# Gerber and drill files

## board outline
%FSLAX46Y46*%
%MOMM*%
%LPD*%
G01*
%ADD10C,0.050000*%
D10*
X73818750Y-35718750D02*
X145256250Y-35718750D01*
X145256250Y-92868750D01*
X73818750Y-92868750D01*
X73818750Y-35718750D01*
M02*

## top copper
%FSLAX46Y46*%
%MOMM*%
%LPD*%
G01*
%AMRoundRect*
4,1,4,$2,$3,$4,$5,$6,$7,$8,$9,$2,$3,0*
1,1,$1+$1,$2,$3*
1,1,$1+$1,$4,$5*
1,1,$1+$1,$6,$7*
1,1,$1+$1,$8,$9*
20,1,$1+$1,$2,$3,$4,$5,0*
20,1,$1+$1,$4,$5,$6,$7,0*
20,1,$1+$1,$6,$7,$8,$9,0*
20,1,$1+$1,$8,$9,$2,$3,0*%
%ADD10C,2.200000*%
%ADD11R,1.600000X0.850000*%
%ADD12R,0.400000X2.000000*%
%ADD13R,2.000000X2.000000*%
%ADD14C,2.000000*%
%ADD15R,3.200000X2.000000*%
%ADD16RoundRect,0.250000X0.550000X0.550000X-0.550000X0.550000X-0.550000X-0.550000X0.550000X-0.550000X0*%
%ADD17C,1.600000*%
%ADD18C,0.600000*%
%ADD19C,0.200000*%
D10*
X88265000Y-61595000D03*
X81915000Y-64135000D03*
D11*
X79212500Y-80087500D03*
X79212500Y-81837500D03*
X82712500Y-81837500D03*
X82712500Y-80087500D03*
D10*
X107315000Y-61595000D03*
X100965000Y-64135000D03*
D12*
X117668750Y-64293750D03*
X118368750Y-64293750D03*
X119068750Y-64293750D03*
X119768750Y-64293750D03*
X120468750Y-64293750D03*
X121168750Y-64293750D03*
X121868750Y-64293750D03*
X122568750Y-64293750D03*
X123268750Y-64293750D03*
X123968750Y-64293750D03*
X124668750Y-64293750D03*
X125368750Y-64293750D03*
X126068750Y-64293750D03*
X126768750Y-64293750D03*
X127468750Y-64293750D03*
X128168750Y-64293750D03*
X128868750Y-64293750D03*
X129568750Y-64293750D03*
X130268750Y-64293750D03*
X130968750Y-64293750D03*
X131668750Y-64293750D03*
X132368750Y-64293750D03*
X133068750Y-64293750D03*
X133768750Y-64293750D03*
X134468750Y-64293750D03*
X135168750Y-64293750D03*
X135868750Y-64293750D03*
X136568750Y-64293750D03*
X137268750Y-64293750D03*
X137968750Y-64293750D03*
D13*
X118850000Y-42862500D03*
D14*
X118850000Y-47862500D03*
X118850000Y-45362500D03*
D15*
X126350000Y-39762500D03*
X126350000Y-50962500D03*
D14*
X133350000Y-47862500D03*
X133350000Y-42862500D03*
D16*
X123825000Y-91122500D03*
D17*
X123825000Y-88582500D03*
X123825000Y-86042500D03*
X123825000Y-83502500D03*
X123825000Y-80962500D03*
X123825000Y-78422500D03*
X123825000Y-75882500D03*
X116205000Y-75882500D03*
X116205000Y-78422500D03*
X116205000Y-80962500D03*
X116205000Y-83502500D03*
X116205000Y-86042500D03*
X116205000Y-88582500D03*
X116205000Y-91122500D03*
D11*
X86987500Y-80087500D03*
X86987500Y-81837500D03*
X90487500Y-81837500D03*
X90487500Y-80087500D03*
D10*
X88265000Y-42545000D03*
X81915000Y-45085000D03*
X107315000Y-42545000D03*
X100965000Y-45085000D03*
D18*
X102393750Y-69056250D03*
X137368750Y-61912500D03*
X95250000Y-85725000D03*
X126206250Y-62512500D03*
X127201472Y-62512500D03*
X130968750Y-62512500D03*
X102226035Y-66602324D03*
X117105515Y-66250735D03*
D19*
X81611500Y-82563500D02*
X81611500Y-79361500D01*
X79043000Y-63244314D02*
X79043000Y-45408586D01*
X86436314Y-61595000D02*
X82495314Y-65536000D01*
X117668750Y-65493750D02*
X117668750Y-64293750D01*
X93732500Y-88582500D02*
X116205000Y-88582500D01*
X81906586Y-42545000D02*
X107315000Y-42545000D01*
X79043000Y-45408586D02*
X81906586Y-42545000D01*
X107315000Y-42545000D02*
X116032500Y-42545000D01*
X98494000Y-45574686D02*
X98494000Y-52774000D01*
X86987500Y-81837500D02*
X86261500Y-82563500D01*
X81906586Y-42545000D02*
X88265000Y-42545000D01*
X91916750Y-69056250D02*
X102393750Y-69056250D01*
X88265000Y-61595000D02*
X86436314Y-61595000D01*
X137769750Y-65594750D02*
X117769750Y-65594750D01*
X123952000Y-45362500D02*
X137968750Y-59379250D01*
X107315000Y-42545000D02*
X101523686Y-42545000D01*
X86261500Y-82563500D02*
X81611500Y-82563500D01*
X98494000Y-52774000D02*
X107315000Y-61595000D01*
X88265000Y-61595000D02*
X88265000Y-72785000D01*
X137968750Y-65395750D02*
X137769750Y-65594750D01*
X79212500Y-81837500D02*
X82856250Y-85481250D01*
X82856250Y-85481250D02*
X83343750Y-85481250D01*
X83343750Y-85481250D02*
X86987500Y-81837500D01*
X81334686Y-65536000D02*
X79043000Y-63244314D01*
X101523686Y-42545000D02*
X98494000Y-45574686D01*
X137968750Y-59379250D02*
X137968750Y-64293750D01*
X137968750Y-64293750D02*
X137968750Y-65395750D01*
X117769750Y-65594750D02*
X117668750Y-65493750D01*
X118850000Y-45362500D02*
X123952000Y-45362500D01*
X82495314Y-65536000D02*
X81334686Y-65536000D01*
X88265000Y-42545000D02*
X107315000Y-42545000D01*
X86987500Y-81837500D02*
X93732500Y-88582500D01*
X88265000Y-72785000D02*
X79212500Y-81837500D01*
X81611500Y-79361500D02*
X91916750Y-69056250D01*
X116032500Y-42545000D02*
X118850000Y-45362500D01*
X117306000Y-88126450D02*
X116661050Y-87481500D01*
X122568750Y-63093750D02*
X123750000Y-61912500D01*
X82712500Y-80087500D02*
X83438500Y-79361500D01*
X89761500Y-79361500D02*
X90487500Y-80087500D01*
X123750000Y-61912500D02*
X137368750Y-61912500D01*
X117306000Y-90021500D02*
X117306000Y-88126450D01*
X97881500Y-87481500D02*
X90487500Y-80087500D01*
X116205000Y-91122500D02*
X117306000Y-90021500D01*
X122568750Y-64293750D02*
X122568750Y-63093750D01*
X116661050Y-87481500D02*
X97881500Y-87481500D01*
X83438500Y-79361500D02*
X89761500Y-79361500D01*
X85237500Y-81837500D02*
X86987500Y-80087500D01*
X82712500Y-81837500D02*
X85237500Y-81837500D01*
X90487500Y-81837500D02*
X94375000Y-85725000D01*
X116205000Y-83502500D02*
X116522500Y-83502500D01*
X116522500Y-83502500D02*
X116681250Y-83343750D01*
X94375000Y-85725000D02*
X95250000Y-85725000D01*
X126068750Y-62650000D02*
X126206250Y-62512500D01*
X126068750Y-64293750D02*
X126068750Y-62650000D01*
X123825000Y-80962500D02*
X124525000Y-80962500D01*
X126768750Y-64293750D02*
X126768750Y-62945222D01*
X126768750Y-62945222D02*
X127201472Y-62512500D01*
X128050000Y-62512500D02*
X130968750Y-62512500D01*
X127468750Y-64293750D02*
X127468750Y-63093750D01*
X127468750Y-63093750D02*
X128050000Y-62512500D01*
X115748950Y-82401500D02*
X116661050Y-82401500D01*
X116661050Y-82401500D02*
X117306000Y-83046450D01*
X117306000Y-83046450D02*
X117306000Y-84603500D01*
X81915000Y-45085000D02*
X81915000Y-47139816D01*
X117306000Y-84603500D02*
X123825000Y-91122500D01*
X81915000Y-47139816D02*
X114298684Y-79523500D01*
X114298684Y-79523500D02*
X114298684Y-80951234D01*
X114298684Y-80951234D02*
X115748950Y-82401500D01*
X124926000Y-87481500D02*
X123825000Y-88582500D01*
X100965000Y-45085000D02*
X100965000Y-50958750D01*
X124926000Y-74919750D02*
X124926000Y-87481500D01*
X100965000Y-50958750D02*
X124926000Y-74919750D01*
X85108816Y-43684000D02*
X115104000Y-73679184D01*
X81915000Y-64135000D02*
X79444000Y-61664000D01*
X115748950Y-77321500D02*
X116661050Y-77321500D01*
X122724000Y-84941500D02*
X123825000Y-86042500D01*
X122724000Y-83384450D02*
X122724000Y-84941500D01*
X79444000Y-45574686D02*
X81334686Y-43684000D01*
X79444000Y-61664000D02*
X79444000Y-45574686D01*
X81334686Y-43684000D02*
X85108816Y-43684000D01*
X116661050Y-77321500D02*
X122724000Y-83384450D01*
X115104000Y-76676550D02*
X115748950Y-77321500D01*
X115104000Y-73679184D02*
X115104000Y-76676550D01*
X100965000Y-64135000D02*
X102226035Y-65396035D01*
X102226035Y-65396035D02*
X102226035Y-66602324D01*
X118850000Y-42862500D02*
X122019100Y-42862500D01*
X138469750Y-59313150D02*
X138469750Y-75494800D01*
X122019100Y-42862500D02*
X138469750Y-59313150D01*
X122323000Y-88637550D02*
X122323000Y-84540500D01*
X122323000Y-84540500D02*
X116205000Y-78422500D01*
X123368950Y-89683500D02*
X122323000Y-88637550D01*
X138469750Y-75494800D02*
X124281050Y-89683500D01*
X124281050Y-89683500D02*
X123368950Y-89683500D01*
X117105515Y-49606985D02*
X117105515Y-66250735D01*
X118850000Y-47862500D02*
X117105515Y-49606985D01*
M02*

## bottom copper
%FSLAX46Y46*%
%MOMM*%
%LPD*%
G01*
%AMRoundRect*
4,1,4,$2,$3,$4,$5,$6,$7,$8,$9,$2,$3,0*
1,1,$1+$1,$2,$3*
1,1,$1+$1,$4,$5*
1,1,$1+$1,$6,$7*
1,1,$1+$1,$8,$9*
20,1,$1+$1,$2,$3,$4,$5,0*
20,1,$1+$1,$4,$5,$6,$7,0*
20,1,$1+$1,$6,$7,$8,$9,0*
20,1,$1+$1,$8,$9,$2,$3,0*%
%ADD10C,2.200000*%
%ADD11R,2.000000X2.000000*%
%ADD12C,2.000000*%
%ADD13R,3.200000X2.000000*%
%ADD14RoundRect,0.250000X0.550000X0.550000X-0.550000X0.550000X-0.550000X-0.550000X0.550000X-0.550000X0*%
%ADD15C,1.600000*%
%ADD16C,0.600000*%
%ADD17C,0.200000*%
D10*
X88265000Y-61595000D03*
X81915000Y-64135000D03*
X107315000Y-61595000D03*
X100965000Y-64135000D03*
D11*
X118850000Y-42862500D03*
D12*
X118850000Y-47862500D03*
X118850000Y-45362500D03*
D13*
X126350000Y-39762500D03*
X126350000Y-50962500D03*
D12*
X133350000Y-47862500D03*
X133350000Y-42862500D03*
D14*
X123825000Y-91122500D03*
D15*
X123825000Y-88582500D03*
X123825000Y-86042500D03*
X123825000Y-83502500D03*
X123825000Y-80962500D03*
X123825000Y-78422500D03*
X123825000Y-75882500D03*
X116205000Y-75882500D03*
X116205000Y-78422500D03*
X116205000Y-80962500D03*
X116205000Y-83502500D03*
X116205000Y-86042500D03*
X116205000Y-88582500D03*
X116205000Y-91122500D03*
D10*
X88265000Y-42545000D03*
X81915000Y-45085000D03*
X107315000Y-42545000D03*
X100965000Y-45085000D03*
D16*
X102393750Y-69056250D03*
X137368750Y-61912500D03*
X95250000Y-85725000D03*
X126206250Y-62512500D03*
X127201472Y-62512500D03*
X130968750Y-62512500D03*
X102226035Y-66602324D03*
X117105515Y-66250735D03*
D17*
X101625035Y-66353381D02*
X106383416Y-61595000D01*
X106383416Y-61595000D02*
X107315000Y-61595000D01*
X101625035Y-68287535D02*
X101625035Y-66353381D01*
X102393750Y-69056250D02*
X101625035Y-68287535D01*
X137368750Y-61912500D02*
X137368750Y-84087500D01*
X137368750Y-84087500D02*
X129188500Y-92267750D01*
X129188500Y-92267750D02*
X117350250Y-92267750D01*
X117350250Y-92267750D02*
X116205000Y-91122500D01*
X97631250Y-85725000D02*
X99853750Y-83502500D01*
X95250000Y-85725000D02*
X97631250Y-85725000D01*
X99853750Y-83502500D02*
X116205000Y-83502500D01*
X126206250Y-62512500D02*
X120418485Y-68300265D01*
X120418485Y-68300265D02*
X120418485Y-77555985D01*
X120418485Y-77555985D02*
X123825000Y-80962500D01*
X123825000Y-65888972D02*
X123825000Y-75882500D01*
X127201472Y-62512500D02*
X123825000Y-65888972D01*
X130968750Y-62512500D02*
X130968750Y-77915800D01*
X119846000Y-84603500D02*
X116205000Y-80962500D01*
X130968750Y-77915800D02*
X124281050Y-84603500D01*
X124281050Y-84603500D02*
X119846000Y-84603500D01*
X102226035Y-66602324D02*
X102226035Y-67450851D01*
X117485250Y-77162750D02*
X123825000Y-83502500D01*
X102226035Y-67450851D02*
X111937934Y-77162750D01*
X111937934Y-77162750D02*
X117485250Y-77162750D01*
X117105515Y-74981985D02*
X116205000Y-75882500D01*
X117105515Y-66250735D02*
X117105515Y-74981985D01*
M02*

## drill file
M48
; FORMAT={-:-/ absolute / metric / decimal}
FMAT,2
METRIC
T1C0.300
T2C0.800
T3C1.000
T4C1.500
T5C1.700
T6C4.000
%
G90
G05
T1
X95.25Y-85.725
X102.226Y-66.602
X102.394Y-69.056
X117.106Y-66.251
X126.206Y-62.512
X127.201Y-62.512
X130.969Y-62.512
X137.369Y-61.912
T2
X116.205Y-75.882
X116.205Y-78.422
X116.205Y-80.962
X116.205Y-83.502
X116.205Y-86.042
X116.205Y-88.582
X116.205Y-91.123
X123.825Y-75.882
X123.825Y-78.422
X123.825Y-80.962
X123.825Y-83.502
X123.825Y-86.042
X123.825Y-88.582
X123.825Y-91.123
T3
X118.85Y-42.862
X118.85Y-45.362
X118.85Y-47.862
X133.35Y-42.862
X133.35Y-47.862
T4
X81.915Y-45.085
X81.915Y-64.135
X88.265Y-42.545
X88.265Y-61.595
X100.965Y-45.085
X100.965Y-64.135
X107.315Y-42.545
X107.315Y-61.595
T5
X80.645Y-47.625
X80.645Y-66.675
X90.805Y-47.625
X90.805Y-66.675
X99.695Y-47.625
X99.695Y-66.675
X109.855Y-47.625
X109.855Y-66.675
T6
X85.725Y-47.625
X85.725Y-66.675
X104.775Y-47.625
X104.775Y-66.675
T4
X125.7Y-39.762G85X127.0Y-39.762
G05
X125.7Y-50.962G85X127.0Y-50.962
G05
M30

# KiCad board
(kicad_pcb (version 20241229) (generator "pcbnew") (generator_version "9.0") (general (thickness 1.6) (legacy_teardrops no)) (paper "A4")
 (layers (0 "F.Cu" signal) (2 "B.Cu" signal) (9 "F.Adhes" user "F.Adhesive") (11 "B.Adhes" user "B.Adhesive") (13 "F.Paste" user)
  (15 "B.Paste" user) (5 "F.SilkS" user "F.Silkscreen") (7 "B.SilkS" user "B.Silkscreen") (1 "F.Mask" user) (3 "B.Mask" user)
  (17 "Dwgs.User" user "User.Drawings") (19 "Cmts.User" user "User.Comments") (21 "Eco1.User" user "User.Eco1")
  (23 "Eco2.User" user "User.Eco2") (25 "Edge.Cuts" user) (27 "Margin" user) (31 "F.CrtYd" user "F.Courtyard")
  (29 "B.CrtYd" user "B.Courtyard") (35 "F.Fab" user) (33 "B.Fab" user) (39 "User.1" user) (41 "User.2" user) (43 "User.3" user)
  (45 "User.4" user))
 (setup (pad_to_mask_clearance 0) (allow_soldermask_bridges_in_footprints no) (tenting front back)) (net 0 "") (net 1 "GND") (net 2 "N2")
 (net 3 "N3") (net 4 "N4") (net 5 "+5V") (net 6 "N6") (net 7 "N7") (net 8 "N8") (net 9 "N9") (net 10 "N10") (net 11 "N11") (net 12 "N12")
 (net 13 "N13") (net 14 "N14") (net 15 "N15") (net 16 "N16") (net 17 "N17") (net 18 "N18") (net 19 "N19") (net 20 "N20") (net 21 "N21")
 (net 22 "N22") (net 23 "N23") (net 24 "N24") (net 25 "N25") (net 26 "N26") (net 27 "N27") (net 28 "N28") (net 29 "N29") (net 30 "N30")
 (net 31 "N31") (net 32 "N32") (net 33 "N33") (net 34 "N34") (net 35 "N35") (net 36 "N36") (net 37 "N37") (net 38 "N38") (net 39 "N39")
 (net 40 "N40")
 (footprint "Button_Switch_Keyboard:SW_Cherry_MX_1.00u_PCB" (layer "F.Cu") (at 88.265 61.595)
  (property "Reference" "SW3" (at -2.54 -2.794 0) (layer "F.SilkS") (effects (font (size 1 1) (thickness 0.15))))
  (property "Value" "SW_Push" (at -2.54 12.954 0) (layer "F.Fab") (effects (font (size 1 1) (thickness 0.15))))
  (pad "" np_thru_hole circle (at -7.62 5.08) (size 1.7 1.7) (drill 1.7) (layers "*.Cu" "*.Mask"))
  (pad "" np_thru_hole circle (at -2.54 5.08) (size 4 4) (drill 4) (layers "*.Cu" "*.Mask"))
  (pad "" np_thru_hole circle (at 2.54 5.08) (size 1.7 1.7) (drill 1.7) (layers "*.Cu" "*.Mask"))
  (pad "1" thru_hole circle (at 0 0) (size 2.2 2.2) (drill 1.5) (layers "*.Cu" "*.Mask") (remove_unused_layers no) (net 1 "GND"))
  (pad "2" thru_hole circle (at -6.35 2.54) (size 2.2 2.2) (drill 1.5) (layers "*.Cu" "*.Mask") (remove_unused_layers no) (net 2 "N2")))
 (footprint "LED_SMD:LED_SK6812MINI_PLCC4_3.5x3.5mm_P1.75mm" (layer "F.Cu") (at 80.9625 80.9625)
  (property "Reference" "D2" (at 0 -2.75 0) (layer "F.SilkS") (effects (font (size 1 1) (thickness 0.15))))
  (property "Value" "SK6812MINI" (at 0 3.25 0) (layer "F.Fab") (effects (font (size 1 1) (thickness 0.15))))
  (pad "1" smd rect (at -1.75 -0.875) (size 1.6 0.85) (layers "F.Cu" "F.Mask" "F.Paste") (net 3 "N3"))
  (pad "2" smd rect (at -1.75 0.875) (size 1.6 0.85) (layers "F.Cu" "F.Mask" "F.Paste") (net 1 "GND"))
  (pad "3" smd rect (at 1.75 0.875) (size 1.6 0.85) (layers "F.Cu" "F.Mask" "F.Paste") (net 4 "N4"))
  (pad "4" smd rect (at 1.75 -0.875) (size 1.6 0.85) (layers "F.Cu" "F.Mask" "F.Paste") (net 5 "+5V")))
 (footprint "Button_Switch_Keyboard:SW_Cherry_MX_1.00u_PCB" (layer "F.Cu") (at 107.315 61.595)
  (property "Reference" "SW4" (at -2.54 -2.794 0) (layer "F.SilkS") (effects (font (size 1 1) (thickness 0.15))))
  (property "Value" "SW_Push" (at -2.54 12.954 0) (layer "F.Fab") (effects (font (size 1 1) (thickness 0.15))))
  (pad "" np_thru_hole circle (at -7.62 5.08) (size 1.7 1.7) (drill 1.7) (layers "*.Cu" "*.Mask"))
  (pad "" np_thru_hole circle (at -2.54 5.08) (size 4 4) (drill 4) (layers "*.Cu" "*.Mask"))
  (pad "" np_thru_hole circle (at 2.54 5.08) (size 1.7 1.7) (drill 1.7) (layers "*.Cu" "*.Mask"))
  (pad "1" thru_hole circle (at 0 0) (size 2.2 2.2) (drill 1.5) (layers "*.Cu" "*.Mask") (remove_unused_layers no) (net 1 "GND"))
  (pad "2" thru_hole circle (at -6.35 2.54) (size 2.2 2.2) (drill 1.5) (layers "*.Cu" "*.Mask") (remove_unused_layers no) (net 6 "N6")))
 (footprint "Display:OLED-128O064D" (layer "F.Cu") (at 127.81875 64.29375)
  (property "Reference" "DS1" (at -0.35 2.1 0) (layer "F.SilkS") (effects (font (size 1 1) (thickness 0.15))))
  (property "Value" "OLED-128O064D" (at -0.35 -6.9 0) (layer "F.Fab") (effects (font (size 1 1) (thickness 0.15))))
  (pad "1" smd rect (at -10.15 0) (size 0.4 2) (layers "F.Cu" "F.Mask" "F.Paste") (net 1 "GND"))
  (pad "2" smd rect (at -9.45 0) (size 0.4 2) (layers "F.Cu" "F.Mask" "F.Paste") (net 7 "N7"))
  (pad "3" smd rect (at -8.75 0) (size 0.4 2) (layers "F.Cu" "F.Mask" "F.Paste") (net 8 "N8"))
  (pad "4" smd rect (at -8.05 0) (size 0.4 2) (layers "F.Cu" "F.Mask" "F.Paste") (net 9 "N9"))
  (pad "5" smd rect (at -7.35 0) (size 0.4 2) (layers "F.Cu" "F.Mask" "F.Paste") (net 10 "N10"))
  (pad "6" smd rect (at -6.65 0) (size 0.4 2) (layers "F.Cu" "F.Mask" "F.Paste") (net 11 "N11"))
  (pad "7" smd rect (at -5.95 0) (size 0.4 2) (layers "F.Cu" "F.Mask" "F.Paste") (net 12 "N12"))
  (pad "8" smd rect (at -5.25 0) (size 0.4 2) (layers "F.Cu" "F.Mask" "F.Paste") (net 5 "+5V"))
  (pad "9" smd rect (at -4.55 0) (size 0.4 2) (layers "F.Cu" "F.Mask" "F.Paste") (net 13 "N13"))
  (pad "10" smd rect (at -3.85 0) (size 0.4 2) (layers "F.Cu" "F.Mask" "F.Paste") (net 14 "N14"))
  (pad "11" smd rect (at -3.15 0) (size 0.4 2) (layers "F.Cu" "F.Mask" "F.Paste") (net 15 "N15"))
  (pad "12" smd rect (at -2.45 0) (size 0.4 2) (layers "F.Cu" "F.Mask" "F.Paste") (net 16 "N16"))
  (pad "13" smd rect (at -1.75 0) (size 0.4 2) (layers "F.Cu" "F.Mask" "F.Paste") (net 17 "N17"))
  (pad "14" smd rect (at -1.05 0) (size 0.4 2) (layers "F.Cu" "F.Mask" "F.Paste") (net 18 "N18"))
  (pad "15" smd rect (at -0.35 0) (size 0.4 2) (layers "F.Cu" "F.Mask" "F.Paste") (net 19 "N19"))
  (pad "16" smd rect (at 0.35 0) (size 0.4 2) (layers "F.Cu" "F.Mask" "F.Paste") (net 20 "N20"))
  (pad "17" smd rect (at 1.05 0) (size 0.4 2) (layers "F.Cu" "F.Mask" "F.Paste") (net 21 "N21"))
  (pad "18" smd rect (at 1.75 0) (size 0.4 2) (layers "F.Cu" "F.Mask" "F.Paste") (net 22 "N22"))
  (pad "19" smd rect (at 2.45 0) (size 0.4 2) (layers "F.Cu" "F.Mask" "F.Paste") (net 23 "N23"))
  (pad "20" smd rect (at 3.15 0) (size 0.4 2) (layers "F.Cu" "F.Mask" "F.Paste") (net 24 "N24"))
  (pad "21" smd rect (at 3.85 0) (size 0.4 2) (layers "F.Cu" "F.Mask" "F.Paste") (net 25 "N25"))
  (pad "22" smd rect (at 4.55 0) (size 0.4 2) (layers "F.Cu" "F.Mask" "F.Paste") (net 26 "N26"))
  (pad "23" smd rect (at 5.25 0) (size 0.4 2) (layers "F.Cu" "F.Mask" "F.Paste") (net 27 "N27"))
  (pad "24" smd rect (at 5.95 0) (size 0.4 2) (layers "F.Cu" "F.Mask" "F.Paste") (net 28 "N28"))
  (pad "25" smd rect (at 6.65 0) (size 0.4 2) (layers "F.Cu" "F.Mask" "F.Paste") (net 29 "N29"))
  (pad "26" smd rect (at 7.35 0) (size 0.4 2) (layers "F.Cu" "F.Mask" "F.Paste") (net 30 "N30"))
  (pad "27" smd rect (at 8.05 0) (size 0.4 2) (layers "F.Cu" "F.Mask" "F.Paste") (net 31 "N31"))
  (pad "28" smd rect (at 8.75 0) (size 0.4 2) (layers "F.Cu" "F.Mask" "F.Paste") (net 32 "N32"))
  (pad "29" smd rect (at 9.45 0) (size 0.4 2) (layers "F.Cu" "F.Mask" "F.Paste") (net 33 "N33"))
  (pad "30" smd rect (at 10.15 0) (size 0.4 2) (layers "F.Cu" "F.Mask" "F.Paste") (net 1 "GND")))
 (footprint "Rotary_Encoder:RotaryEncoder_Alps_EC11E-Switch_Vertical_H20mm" (layer "F.Cu") (at 118.85 42.8625)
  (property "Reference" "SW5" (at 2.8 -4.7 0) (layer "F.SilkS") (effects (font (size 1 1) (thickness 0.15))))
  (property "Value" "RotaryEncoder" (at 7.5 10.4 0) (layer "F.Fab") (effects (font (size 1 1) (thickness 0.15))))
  (pad "A" thru_hole rect (at 0 0) (size 2 2) (drill 1) (layers "*.Cu" "*.Mask") (remove_unused_layers no) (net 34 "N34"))
  (pad "B" thru_hole circle (at 0 5) (size 2 2) (drill 1) (layers "*.Cu" "*.Mask") (remove_unused_layers no) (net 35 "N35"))
  (pad "C" thru_hole circle (at 0 2.5) (size 2 2) (drill 1) (layers "*.Cu" "*.Mask") (remove_unused_layers no) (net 1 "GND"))
  (pad "MP" thru_hole rect (at 7.5 -3.1) (size 3.2 2) (drill oval 2.8 1.5) (layers "*.Cu" "*.Mask") (remove_unused_layers no))
  (pad "MP" thru_hole rect (at 7.5 8.1) (size 3.2 2) (drill oval 2.8 1.5) (layers "*.Cu" "*.Mask") (remove_unused_layers no))
  (pad "S1" thru_hole circle (at 14.5 5) (size 2 2) (drill 1) (layers "*.Cu" "*.Mask") (remove_unused_layers no))
  (pad "S2" thru_hole circle (at 14.5 0) (size 2 2) (drill 1) (layers "*.Cu" "*.Mask") (remove_unused_layers no)))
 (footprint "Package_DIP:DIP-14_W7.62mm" (layer "F.Cu") (at 123.825 91.1225 180)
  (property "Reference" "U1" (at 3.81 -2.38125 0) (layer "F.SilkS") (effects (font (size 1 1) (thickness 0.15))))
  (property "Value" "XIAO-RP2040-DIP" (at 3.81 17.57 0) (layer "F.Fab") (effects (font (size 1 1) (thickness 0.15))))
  (pad "1" thru_hole roundrect (at 0 0 180) (size 1.6 1.6) (drill 0.8) (layers "*.Cu" "*.Mask") (remove_unused_layers no)
   (roundrect_rratio 0.15625) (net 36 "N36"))
  (pad "2" thru_hole circle (at 0 2.54 180) (size 1.6 1.6) (drill 0.8) (layers "*.Cu" "*.Mask") (remove_unused_layers no) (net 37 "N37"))
  (pad "3" thru_hole circle (at 0 5.08 180) (size 1.6 1.6) (drill 0.8) (layers "*.Cu" "*.Mask") (remove_unused_layers no) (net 2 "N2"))
  (pad "4" thru_hole circle (at 0 7.62 180) (size 1.6 1.6) (drill 0.8) (layers "*.Cu" "*.Mask") (remove_unused_layers no) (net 6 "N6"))
  (pad "5" thru_hole circle (at 0 10.16 180) (size 1.6 1.6) (drill 0.8) (layers "*.Cu" "*.Mask") (remove_unused_layers no) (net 17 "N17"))
  (pad "6" thru_hole circle (at 0 12.7 180) (size 1.6 1.6) (drill 0.8) (layers "*.Cu" "*.Mask") (remove_unused_layers no) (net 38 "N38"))
  (pad "7" thru_hole circle (at 0 15.24 180) (size 1.6 1.6) (drill 0.8) (layers "*.Cu" "*.Mask") (remove_unused_layers no) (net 18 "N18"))
  (pad "8" thru_hole circle (at 7.62 15.24 180) (size 1.6 1.6) (drill 0.8) (layers "*.Cu" "*.Mask") (remove_unused_layers no) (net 35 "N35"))
  (pad "9" thru_hole circle (at 7.62 12.7 180) (size 1.6 1.6) (drill 0.8) (layers "*.Cu" "*.Mask") (remove_unused_layers no) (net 34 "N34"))
  (pad "10" thru_hole circle (at 7.62 10.16 180) (size 1.6 1.6) (drill 0.8) (layers "*.Cu" "*.Mask") (remove_unused_layers no)
   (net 19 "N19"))
  (pad "11" thru_hole circle (at 7.62 7.62 180) (size 1.6 1.6) (drill 0.8) (layers "*.Cu" "*.Mask") (remove_unused_layers no) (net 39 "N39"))
  (pad "12" thru_hole circle (at 7.62 5.08 180) (size 1.6 1.6) (drill 0.8) (layers "*.Cu" "*.Mask") (remove_unused_layers no) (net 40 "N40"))
  (pad "13" thru_hole circle (at 7.62 2.54 180) (size 1.6 1.6) (drill 0.8) (layers "*.Cu" "*.Mask") (remove_unused_layers no) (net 1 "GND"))
  (pad "14" thru_hole circle (at 7.62 0 180) (size 1.6 1.6) (drill 0.8) (layers "*.Cu" "*.Mask") (remove_unused_layers no) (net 5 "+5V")))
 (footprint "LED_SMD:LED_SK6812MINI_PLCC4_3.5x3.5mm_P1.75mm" (layer "F.Cu") (at 88.7375 80.9625)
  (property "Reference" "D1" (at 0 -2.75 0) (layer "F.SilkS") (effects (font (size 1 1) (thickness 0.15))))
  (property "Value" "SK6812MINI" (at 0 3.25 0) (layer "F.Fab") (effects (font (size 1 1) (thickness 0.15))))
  (pad "1" smd rect (at -1.75 -0.875) (size 1.6 0.85) (layers "F.Cu" "F.Mask" "F.Paste") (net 4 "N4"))
  (pad "2" smd rect (at -1.75 0.875) (size 1.6 0.85) (layers "F.Cu" "F.Mask" "F.Paste") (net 1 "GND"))
  (pad "3" smd rect (at 1.75 0.875) (size 1.6 0.85) (layers "F.Cu" "F.Mask" "F.Paste") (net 39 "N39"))
  (pad "4" smd rect (at 1.75 -0.875) (size 1.6 0.85) (layers "F.Cu" "F.Mask" "F.Paste") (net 5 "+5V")))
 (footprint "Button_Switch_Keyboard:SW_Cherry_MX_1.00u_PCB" (layer "F.Cu") (at 88.265 42.545)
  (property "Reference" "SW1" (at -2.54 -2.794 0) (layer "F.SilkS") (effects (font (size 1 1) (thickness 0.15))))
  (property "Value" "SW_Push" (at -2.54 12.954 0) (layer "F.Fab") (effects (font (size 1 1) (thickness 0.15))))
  (pad "" np_thru_hole circle (at -7.62 5.08) (size 1.7 1.7) (drill 1.7) (layers "*.Cu" "*.Mask"))
  (pad "" np_thru_hole circle (at -2.54 5.08) (size 4 4) (drill 4) (layers "*.Cu" "*.Mask"))
  (pad "" np_thru_hole circle (at 2.54 5.08) (size 1.7 1.7) (drill 1.7) (layers "*.Cu" "*.Mask"))
  (pad "1" thru_hole circle (at 0 0) (size 2.2 2.2) (drill 1.5) (layers "*.Cu" "*.Mask") (remove_unused_layers no) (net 1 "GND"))
  (pad "2" thru_hole circle (at -6.35 2.54) (size 2.2 2.2) (drill 1.5) (layers "*.Cu" "*.Mask") (remove_unused_layers no) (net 36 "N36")))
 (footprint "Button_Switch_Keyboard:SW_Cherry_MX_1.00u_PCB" (layer "F.Cu") (at 107.315 42.545)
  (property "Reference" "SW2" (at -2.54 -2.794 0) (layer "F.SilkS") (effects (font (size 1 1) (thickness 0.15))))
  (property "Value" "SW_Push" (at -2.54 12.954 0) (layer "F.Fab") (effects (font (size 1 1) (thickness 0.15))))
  (pad "" np_thru_hole circle (at -7.62 5.08) (size 1.7 1.7) (drill 1.7) (layers "*.Cu" "*.Mask"))
  (pad "" np_thru_hole circle (at -2.54 5.08) (size 4 4) (drill 4) (layers "*.Cu" "*.Mask"))
  (pad "" np_thru_hole circle (at 2.54 5.08) (size 1.7 1.7) (drill 1.7) (layers "*.Cu" "*.Mask"))
  (pad "1" thru_hole circle (at 0 0) (size 2.2 2.2) (drill 1.5) (layers "*.Cu" "*.Mask") (remove_unused_layers no) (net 1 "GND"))
  (pad "2" thru_hole circle (at -6.35 2.54) (size 2.2 2.2) (drill 1.5) (layers "*.Cu" "*.Mask") (remove_unused_layers no) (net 37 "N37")))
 (gr_rect (start 73.81875 35.71875) (end 145.25625 92.86875) (stroke (width 0.05) (type default)) (fill no) (layer "Edge.Cuts"))
 (segment (start 81.6115 82.5635) (end 81.6115 79.3615) (width 0.2) (layer "F.Cu") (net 1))
 (segment (start 79.043 63.244314) (end 79.043 45.408586) (width 0.2) (layer "F.Cu") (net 1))
 (segment (start 86.436314 61.595) (end 82.495314 65.536) (width 0.2) (layer "F.Cu") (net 1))
 (segment (start 117.66875 65.49375) (end 117.66875 64.29375) (width 0.2) (layer "F.Cu") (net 1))
 (segment (start 93.7325 88.5825) (end 116.205 88.5825) (width 0.2) (layer "F.Cu") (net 1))
 (segment (start 81.906586 42.545) (end 107.315 42.545) (width 0.2) (layer "F.Cu") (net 1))
 (segment (start 79.043 45.408586) (end 81.906586 42.545) (width 0.2) (layer "F.Cu") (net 1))
 (segment (start 107.315 42.545) (end 116.0325 42.545) (width 0.2) (layer "F.Cu") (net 1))
 (segment (start 98.494 45.574686) (end 98.494 52.774) (width 0.2) (layer "F.Cu") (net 1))
 (segment (start 86.9875 81.8375) (end 86.2615 82.5635) (width 0.2) (layer "F.Cu") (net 1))
 (segment (start 81.906586 42.545) (end 88.265 42.545) (width 0.2) (layer "F.Cu") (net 1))
 (segment (start 91.91675 69.05625) (end 102.39375 69.05625) (width 0.2) (layer "F.Cu") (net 1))
 (segment (start 88.265 61.595) (end 86.436314 61.595) (width 0.2) (layer "F.Cu") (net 1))
 (segment (start 137.76975 65.59475) (end 117.76975 65.59475) (width 0.2) (layer "F.Cu") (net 1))
 (segment (start 123.952 45.3625) (end 137.96875 59.37925) (width 0.2) (layer "F.Cu") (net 1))
 (segment (start 107.315 42.545) (end 101.523686 42.545) (width 0.2) (layer "F.Cu") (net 1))
 (segment (start 86.2615 82.5635) (end 81.6115 82.5635) (width 0.2) (layer "F.Cu") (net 1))
 (segment (start 98.494 52.774) (end 107.315 61.595) (width 0.2) (layer "F.Cu") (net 1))
 (segment (start 88.265 61.595) (end 88.265 72.785) (width 0.2) (layer "F.Cu") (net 1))
 (segment (start 137.96875 65.39575) (end 137.76975 65.59475) (width 0.2) (layer "F.Cu") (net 1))
 (segment (start 79.2125 81.8375) (end 82.85625 85.48125) (width 0.2) (layer "F.Cu") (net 1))
 (segment (start 82.85625 85.48125) (end 83.34375 85.48125) (width 0.2) (layer "F.Cu") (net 1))
 (segment (start 83.34375 85.48125) (end 86.9875 81.8375) (width 0.2) (layer "F.Cu") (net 1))
 (segment (start 81.334686 65.536) (end 79.043 63.244314) (width 0.2) (layer "F.Cu") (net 1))
 (segment (start 101.523686 42.545) (end 98.494 45.574686) (width 0.2) (layer "F.Cu") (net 1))
 (segment (start 137.96875 59.37925) (end 137.96875 64.29375) (width 0.2) (layer "F.Cu") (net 1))
 (segment (start 137.96875 64.29375) (end 137.96875 65.39575) (width 0.2) (layer "F.Cu") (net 1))
 (segment (start 117.76975 65.59475) (end 117.66875 65.49375) (width 0.2) (layer "F.Cu") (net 1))
 (segment (start 118.85 45.3625) (end 123.952 45.3625) (width 0.2) (layer "F.Cu") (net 1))
 (segment (start 82.495314 65.536) (end 81.334686 65.536) (width 0.2) (layer "F.Cu") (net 1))
 (segment (start 88.265 42.545) (end 107.315 42.545) (width 0.2) (layer "F.Cu") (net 1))
 (segment (start 86.9875 81.8375) (end 93.7325 88.5825) (width 0.2) (layer "F.Cu") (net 1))
 (segment (start 88.265 72.785) (end 79.2125 81.8375) (width 0.2) (layer "F.Cu") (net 1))
 (segment (start 81.6115 79.3615) (end 91.91675 69.05625) (width 0.2) (layer "F.Cu") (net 1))
 (segment (start 116.0325 42.545) (end 118.85 45.3625) (width 0.2) (layer "F.Cu") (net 1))
 (via (at 102.39375 69.05625) (size 0.6) (drill 0.3) (layers "F.Cu" "B.Cu") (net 1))
 (segment (start 101.625035 66.353381) (end 106.383416 61.595) (width 0.2) (layer "B.Cu") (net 1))
 (segment (start 106.383416 61.595) (end 107.315 61.595) (width 0.2) (layer "B.Cu") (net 1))
 (segment (start 101.625035 68.287535) (end 101.625035 66.353381) (width 0.2) (layer "B.Cu") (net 1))
 (segment (start 102.39375 69.05625) (end 101.625035 68.287535) (width 0.2) (layer "B.Cu") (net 1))
 (segment (start 117.306 88.12645) (end 116.66105 87.4815) (width 0.2) (layer "F.Cu") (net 5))
 (segment (start 122.56875 63.09375) (end 123.75 61.9125) (width 0.2) (layer "F.Cu") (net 5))
 (segment (start 82.7125 80.0875) (end 83.4385 79.3615) (width 0.2) (layer "F.Cu") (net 5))
 (segment (start 89.7615 79.3615) (end 90.4875 80.0875) (width 0.2) (layer "F.Cu") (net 5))
 (segment (start 123.75 61.9125) (end 137.36875 61.9125) (width 0.2) (layer "F.Cu") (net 5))
 (segment (start 117.306 90.0215) (end 117.306 88.12645) (width 0.2) (layer "F.Cu") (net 5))
 (segment (start 97.8815 87.4815) (end 90.4875 80.0875) (width 0.2) (layer "F.Cu") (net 5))
 (segment (start 116.205 91.1225) (end 117.306 90.0215) (width 0.2) (layer "F.Cu") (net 5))
 (segment (start 122.56875 64.29375) (end 122.56875 63.09375) (width 0.2) (layer "F.Cu") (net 5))
 (segment (start 116.66105 87.4815) (end 97.8815 87.4815) (width 0.2) (layer "F.Cu") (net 5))
 (segment (start 83.4385 79.3615) (end 89.7615 79.3615) (width 0.2) (layer "F.Cu") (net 5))
 (via (at 137.36875 61.9125) (size 0.6) (drill 0.3) (layers "F.Cu" "B.Cu") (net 5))
 (segment (start 137.36875 61.9125) (end 137.36875 84.0875) (width 0.2) (layer "B.Cu") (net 5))
 (segment (start 137.36875 84.0875) (end 129.1885 92.26775) (width 0.2) (layer "B.Cu") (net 5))
 (segment (start 129.1885 92.26775) (end 117.35025 92.26775) (width 0.2) (layer "B.Cu") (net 5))
 (segment (start 117.35025 92.26775) (end 116.205 91.1225) (width 0.2) (layer "B.Cu") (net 5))
 (segment (start 85.2375 81.8375) (end 86.9875 80.0875) (width 0.2) (layer "F.Cu") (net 4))
 (segment (start 82.7125 81.8375) (end 85.2375 81.8375) (width 0.2) (layer "F.Cu") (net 4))
 (segment (start 90.4875 81.8375) (end 94.375 85.725) (width 0.2) (layer "F.Cu") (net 39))
 (segment (start 116.205 83.5025) (end 116.5225 83.5025) (width 0.2) (layer "F.Cu") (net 39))
 (segment (start 116.5225 83.5025) (end 116.68125 83.34375) (width 0.2) (layer "F.Cu") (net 39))
 (segment (start 94.375 85.725) (end 95.25 85.725) (width 0.2) (layer "F.Cu") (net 39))
 (via (at 95.25 85.725) (size 0.6) (drill 0.3) (layers "F.Cu" "B.Cu") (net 39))
 (segment (start 97.63125 85.725) (end 99.85375 83.5025) (width 0.2) (layer "B.Cu") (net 39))
 (segment (start 95.25 85.725) (end 97.63125 85.725) (width 0.2) (layer "B.Cu") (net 39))
 (segment (start 99.85375 83.5025) (end 116.205 83.5025) (width 0.2) (layer "B.Cu") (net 39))
 (segment (start 126.06875 62.65) (end 126.20625 62.5125) (width 0.2) (layer "F.Cu") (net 17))
 (segment (start 126.06875 64.29375) (end 126.06875 62.65) (width 0.2) (layer "F.Cu") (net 17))
 (segment (start 123.825 80.9625) (end 124.525 80.9625) (width 0.2) (layer "F.Cu") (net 17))
 (via (at 126.20625 62.5125) (size 0.6) (drill 0.3) (layers "F.Cu" "B.Cu") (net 17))
 (segment (start 126.20625 62.5125) (end 120.418485 68.300265) (width 0.2) (layer "B.Cu") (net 17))
 (segment (start 120.418485 68.300265) (end 120.418485 77.555985) (width 0.2) (layer "B.Cu") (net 17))
 (segment (start 120.418485 77.555985) (end 123.825 80.9625) (width 0.2) (layer "B.Cu") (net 17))
 (segment (start 126.76875 64.29375) (end 126.76875 62.945222) (width 0.2) (layer "F.Cu") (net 18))
 (segment (start 126.76875 62.945222) (end 127.201472 62.5125) (width 0.2) (layer "F.Cu") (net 18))
 (via (at 127.201472 62.5125) (size 0.6) (drill 0.3) (layers "F.Cu" "B.Cu") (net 18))
 (segment (start 123.825 65.888972) (end 123.825 75.8825) (width 0.2) (layer "B.Cu") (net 18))
 (segment (start 127.201472 62.5125) (end 123.825 65.888972) (width 0.2) (layer "B.Cu") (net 18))
 (segment (start 128.05 62.5125) (end 130.96875 62.5125) (width 0.2) (layer "F.Cu") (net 19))
 (segment (start 127.46875 64.29375) (end 127.46875 63.09375) (width 0.2) (layer "F.Cu") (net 19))
 (segment (start 127.46875 63.09375) (end 128.05 62.5125) (width 0.2) (layer "F.Cu") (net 19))
 (via (at 130.96875 62.5125) (size 0.6) (drill 0.3) (layers "F.Cu" "B.Cu") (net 19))
 (segment (start 130.96875 62.5125) (end 130.96875 77.9158) (width 0.2) (layer "B.Cu") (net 19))
 (segment (start 119.846 84.6035) (end 116.205 80.9625) (width 0.2) (layer "B.Cu") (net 19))
 (segment (start 130.96875 77.9158) (end 124.28105 84.6035) (width 0.2) (layer "B.Cu") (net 19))
 (segment (start 124.28105 84.6035) (end 119.846 84.6035) (width 0.2) (layer "B.Cu") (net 19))
 (segment (start 115.74895 82.4015) (end 116.66105 82.4015) (width 0.2) (layer "F.Cu") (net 36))
 (segment (start 116.66105 82.4015) (end 117.306 83.04645) (width 0.2) (layer "F.Cu") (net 36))
 (segment (start 117.306 83.04645) (end 117.306 84.6035) (width 0.2) (layer "F.Cu") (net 36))
 (segment (start 81.915 45.085) (end 81.915 47.139816) (width 0.2) (layer "F.Cu") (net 36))
 (segment (start 117.306 84.6035) (end 123.825 91.1225) (width 0.2) (layer "F.Cu") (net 36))
 (segment (start 81.915 47.139816) (end 114.298684 79.5235) (width 0.2) (layer "F.Cu") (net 36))
 (segment (start 114.298684 79.5235) (end 114.298684 80.951234) (width 0.2) (layer "F.Cu") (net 36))
 (segment (start 114.298684 80.951234) (end 115.74895 82.4015) (width 0.2) (layer "F.Cu") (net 36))
 (segment (start 124.926 87.4815) (end 123.825 88.5825) (width 0.2) (layer "F.Cu") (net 37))
 (segment (start 100.965 45.085) (end 100.965 50.95875) (width 0.2) (layer "F.Cu") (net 37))
 (segment (start 124.926 74.91975) (end 124.926 87.4815) (width 0.2) (layer "F.Cu") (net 37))
 (segment (start 100.965 50.95875) (end 124.926 74.91975) (width 0.2) (layer "F.Cu") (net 37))
 (segment (start 85.108816 43.684) (end 115.104 73.679184) (width 0.2) (layer "F.Cu") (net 2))
 (segment (start 81.915 64.135) (end 79.444 61.664) (width 0.2) (layer "F.Cu") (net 2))
 (segment (start 115.74895 77.3215) (end 116.66105 77.3215) (width 0.2) (layer "F.Cu") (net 2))
 (segment (start 122.724 84.9415) (end 123.825 86.0425) (width 0.2) (layer "F.Cu") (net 2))
 (segment (start 122.724 83.38445) (end 122.724 84.9415) (width 0.2) (layer "F.Cu") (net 2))
 (segment (start 79.444 45.574686) (end 81.334686 43.684) (width 0.2) (layer "F.Cu") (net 2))
 (segment (start 79.444 61.664) (end 79.444 45.574686) (width 0.2) (layer "F.Cu") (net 2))
 (segment (start 81.334686 43.684) (end 85.108816 43.684) (width 0.2) (layer "F.Cu") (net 2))
 (segment (start 116.66105 77.3215) (end 122.724 83.38445) (width 0.2) (layer "F.Cu") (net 2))
 (segment (start 115.104 76.67655) (end 115.74895 77.3215) (width 0.2) (layer "F.Cu") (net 2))
 (segment (start 115.104 73.679184) (end 115.104 76.67655) (width 0.2) (layer "F.Cu") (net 2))
 (segment (start 100.965 64.135) (end 102.226035 65.396035) (width 0.2) (layer "F.Cu") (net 6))
 (segment (start 102.226035 65.396035) (end 102.226035 66.602324) (width 0.2) (layer "F.Cu") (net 6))
 (via (at 102.226035 66.602324) (size 0.6) (drill 0.3) (layers "F.Cu" "B.Cu") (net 6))
 (segment (start 102.226035 66.602324) (end 102.226035 67.450851) (width 0.2) (layer "B.Cu") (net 6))
 (segment (start 117.48525 77.16275) (end 123.825 83.5025) (width 0.2) (layer "B.Cu") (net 6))
 (segment (start 102.226035 67.450851) (end 111.937934 77.16275) (width 0.2) (layer "B.Cu") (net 6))
 (segment (start 111.937934 77.16275) (end 117.48525 77.16275) (width 0.2) (layer "B.Cu") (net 6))
 (segment (start 118.85 42.8625) (end 122.0191 42.8625) (width 0.2) (layer "F.Cu") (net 34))
 (segment (start 138.46975 59.31315) (end 138.46975 75.4948) (width 0.2) (layer "F.Cu") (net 34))
 (segment (start 122.0191 42.8625) (end 138.46975 59.31315) (width 0.2) (layer "F.Cu") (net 34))
 (segment (start 122.323 88.63755) (end 122.323 84.5405) (width 0.2) (layer "F.Cu") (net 34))
 (segment (start 122.323 84.5405) (end 116.205 78.4225) (width 0.2) (layer "F.Cu") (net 34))
 (segment (start 123.36895 89.6835) (end 122.323 88.63755) (width 0.2) (layer "F.Cu") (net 34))
 (segment (start 138.46975 75.4948) (end 124.28105 89.6835) (width 0.2) (layer "F.Cu") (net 34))
 (segment (start 124.28105 89.6835) (end 123.36895 89.6835) (width 0.2) (layer "F.Cu") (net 34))
 (segment (start 117.105515 49.606985) (end 117.105515 66.250735) (width 0.2) (layer "F.Cu") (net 35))
 (segment (start 118.85 47.8625) (end 117.105515 49.606985) (width 0.2) (layer "F.Cu") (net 35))
 (via (at 117.105515 66.250735) (size 0.6) (drill 0.3) (layers "F.Cu" "B.Cu") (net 35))
 (segment (start 117.105515 74.981985) (end 116.205 75.8825) (width 0.2) (layer "B.Cu") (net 35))
 (segment (start 117.105515 66.250735) (end 117.105515 74.981985) (width 0.2) (layer "B.Cu") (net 35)))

